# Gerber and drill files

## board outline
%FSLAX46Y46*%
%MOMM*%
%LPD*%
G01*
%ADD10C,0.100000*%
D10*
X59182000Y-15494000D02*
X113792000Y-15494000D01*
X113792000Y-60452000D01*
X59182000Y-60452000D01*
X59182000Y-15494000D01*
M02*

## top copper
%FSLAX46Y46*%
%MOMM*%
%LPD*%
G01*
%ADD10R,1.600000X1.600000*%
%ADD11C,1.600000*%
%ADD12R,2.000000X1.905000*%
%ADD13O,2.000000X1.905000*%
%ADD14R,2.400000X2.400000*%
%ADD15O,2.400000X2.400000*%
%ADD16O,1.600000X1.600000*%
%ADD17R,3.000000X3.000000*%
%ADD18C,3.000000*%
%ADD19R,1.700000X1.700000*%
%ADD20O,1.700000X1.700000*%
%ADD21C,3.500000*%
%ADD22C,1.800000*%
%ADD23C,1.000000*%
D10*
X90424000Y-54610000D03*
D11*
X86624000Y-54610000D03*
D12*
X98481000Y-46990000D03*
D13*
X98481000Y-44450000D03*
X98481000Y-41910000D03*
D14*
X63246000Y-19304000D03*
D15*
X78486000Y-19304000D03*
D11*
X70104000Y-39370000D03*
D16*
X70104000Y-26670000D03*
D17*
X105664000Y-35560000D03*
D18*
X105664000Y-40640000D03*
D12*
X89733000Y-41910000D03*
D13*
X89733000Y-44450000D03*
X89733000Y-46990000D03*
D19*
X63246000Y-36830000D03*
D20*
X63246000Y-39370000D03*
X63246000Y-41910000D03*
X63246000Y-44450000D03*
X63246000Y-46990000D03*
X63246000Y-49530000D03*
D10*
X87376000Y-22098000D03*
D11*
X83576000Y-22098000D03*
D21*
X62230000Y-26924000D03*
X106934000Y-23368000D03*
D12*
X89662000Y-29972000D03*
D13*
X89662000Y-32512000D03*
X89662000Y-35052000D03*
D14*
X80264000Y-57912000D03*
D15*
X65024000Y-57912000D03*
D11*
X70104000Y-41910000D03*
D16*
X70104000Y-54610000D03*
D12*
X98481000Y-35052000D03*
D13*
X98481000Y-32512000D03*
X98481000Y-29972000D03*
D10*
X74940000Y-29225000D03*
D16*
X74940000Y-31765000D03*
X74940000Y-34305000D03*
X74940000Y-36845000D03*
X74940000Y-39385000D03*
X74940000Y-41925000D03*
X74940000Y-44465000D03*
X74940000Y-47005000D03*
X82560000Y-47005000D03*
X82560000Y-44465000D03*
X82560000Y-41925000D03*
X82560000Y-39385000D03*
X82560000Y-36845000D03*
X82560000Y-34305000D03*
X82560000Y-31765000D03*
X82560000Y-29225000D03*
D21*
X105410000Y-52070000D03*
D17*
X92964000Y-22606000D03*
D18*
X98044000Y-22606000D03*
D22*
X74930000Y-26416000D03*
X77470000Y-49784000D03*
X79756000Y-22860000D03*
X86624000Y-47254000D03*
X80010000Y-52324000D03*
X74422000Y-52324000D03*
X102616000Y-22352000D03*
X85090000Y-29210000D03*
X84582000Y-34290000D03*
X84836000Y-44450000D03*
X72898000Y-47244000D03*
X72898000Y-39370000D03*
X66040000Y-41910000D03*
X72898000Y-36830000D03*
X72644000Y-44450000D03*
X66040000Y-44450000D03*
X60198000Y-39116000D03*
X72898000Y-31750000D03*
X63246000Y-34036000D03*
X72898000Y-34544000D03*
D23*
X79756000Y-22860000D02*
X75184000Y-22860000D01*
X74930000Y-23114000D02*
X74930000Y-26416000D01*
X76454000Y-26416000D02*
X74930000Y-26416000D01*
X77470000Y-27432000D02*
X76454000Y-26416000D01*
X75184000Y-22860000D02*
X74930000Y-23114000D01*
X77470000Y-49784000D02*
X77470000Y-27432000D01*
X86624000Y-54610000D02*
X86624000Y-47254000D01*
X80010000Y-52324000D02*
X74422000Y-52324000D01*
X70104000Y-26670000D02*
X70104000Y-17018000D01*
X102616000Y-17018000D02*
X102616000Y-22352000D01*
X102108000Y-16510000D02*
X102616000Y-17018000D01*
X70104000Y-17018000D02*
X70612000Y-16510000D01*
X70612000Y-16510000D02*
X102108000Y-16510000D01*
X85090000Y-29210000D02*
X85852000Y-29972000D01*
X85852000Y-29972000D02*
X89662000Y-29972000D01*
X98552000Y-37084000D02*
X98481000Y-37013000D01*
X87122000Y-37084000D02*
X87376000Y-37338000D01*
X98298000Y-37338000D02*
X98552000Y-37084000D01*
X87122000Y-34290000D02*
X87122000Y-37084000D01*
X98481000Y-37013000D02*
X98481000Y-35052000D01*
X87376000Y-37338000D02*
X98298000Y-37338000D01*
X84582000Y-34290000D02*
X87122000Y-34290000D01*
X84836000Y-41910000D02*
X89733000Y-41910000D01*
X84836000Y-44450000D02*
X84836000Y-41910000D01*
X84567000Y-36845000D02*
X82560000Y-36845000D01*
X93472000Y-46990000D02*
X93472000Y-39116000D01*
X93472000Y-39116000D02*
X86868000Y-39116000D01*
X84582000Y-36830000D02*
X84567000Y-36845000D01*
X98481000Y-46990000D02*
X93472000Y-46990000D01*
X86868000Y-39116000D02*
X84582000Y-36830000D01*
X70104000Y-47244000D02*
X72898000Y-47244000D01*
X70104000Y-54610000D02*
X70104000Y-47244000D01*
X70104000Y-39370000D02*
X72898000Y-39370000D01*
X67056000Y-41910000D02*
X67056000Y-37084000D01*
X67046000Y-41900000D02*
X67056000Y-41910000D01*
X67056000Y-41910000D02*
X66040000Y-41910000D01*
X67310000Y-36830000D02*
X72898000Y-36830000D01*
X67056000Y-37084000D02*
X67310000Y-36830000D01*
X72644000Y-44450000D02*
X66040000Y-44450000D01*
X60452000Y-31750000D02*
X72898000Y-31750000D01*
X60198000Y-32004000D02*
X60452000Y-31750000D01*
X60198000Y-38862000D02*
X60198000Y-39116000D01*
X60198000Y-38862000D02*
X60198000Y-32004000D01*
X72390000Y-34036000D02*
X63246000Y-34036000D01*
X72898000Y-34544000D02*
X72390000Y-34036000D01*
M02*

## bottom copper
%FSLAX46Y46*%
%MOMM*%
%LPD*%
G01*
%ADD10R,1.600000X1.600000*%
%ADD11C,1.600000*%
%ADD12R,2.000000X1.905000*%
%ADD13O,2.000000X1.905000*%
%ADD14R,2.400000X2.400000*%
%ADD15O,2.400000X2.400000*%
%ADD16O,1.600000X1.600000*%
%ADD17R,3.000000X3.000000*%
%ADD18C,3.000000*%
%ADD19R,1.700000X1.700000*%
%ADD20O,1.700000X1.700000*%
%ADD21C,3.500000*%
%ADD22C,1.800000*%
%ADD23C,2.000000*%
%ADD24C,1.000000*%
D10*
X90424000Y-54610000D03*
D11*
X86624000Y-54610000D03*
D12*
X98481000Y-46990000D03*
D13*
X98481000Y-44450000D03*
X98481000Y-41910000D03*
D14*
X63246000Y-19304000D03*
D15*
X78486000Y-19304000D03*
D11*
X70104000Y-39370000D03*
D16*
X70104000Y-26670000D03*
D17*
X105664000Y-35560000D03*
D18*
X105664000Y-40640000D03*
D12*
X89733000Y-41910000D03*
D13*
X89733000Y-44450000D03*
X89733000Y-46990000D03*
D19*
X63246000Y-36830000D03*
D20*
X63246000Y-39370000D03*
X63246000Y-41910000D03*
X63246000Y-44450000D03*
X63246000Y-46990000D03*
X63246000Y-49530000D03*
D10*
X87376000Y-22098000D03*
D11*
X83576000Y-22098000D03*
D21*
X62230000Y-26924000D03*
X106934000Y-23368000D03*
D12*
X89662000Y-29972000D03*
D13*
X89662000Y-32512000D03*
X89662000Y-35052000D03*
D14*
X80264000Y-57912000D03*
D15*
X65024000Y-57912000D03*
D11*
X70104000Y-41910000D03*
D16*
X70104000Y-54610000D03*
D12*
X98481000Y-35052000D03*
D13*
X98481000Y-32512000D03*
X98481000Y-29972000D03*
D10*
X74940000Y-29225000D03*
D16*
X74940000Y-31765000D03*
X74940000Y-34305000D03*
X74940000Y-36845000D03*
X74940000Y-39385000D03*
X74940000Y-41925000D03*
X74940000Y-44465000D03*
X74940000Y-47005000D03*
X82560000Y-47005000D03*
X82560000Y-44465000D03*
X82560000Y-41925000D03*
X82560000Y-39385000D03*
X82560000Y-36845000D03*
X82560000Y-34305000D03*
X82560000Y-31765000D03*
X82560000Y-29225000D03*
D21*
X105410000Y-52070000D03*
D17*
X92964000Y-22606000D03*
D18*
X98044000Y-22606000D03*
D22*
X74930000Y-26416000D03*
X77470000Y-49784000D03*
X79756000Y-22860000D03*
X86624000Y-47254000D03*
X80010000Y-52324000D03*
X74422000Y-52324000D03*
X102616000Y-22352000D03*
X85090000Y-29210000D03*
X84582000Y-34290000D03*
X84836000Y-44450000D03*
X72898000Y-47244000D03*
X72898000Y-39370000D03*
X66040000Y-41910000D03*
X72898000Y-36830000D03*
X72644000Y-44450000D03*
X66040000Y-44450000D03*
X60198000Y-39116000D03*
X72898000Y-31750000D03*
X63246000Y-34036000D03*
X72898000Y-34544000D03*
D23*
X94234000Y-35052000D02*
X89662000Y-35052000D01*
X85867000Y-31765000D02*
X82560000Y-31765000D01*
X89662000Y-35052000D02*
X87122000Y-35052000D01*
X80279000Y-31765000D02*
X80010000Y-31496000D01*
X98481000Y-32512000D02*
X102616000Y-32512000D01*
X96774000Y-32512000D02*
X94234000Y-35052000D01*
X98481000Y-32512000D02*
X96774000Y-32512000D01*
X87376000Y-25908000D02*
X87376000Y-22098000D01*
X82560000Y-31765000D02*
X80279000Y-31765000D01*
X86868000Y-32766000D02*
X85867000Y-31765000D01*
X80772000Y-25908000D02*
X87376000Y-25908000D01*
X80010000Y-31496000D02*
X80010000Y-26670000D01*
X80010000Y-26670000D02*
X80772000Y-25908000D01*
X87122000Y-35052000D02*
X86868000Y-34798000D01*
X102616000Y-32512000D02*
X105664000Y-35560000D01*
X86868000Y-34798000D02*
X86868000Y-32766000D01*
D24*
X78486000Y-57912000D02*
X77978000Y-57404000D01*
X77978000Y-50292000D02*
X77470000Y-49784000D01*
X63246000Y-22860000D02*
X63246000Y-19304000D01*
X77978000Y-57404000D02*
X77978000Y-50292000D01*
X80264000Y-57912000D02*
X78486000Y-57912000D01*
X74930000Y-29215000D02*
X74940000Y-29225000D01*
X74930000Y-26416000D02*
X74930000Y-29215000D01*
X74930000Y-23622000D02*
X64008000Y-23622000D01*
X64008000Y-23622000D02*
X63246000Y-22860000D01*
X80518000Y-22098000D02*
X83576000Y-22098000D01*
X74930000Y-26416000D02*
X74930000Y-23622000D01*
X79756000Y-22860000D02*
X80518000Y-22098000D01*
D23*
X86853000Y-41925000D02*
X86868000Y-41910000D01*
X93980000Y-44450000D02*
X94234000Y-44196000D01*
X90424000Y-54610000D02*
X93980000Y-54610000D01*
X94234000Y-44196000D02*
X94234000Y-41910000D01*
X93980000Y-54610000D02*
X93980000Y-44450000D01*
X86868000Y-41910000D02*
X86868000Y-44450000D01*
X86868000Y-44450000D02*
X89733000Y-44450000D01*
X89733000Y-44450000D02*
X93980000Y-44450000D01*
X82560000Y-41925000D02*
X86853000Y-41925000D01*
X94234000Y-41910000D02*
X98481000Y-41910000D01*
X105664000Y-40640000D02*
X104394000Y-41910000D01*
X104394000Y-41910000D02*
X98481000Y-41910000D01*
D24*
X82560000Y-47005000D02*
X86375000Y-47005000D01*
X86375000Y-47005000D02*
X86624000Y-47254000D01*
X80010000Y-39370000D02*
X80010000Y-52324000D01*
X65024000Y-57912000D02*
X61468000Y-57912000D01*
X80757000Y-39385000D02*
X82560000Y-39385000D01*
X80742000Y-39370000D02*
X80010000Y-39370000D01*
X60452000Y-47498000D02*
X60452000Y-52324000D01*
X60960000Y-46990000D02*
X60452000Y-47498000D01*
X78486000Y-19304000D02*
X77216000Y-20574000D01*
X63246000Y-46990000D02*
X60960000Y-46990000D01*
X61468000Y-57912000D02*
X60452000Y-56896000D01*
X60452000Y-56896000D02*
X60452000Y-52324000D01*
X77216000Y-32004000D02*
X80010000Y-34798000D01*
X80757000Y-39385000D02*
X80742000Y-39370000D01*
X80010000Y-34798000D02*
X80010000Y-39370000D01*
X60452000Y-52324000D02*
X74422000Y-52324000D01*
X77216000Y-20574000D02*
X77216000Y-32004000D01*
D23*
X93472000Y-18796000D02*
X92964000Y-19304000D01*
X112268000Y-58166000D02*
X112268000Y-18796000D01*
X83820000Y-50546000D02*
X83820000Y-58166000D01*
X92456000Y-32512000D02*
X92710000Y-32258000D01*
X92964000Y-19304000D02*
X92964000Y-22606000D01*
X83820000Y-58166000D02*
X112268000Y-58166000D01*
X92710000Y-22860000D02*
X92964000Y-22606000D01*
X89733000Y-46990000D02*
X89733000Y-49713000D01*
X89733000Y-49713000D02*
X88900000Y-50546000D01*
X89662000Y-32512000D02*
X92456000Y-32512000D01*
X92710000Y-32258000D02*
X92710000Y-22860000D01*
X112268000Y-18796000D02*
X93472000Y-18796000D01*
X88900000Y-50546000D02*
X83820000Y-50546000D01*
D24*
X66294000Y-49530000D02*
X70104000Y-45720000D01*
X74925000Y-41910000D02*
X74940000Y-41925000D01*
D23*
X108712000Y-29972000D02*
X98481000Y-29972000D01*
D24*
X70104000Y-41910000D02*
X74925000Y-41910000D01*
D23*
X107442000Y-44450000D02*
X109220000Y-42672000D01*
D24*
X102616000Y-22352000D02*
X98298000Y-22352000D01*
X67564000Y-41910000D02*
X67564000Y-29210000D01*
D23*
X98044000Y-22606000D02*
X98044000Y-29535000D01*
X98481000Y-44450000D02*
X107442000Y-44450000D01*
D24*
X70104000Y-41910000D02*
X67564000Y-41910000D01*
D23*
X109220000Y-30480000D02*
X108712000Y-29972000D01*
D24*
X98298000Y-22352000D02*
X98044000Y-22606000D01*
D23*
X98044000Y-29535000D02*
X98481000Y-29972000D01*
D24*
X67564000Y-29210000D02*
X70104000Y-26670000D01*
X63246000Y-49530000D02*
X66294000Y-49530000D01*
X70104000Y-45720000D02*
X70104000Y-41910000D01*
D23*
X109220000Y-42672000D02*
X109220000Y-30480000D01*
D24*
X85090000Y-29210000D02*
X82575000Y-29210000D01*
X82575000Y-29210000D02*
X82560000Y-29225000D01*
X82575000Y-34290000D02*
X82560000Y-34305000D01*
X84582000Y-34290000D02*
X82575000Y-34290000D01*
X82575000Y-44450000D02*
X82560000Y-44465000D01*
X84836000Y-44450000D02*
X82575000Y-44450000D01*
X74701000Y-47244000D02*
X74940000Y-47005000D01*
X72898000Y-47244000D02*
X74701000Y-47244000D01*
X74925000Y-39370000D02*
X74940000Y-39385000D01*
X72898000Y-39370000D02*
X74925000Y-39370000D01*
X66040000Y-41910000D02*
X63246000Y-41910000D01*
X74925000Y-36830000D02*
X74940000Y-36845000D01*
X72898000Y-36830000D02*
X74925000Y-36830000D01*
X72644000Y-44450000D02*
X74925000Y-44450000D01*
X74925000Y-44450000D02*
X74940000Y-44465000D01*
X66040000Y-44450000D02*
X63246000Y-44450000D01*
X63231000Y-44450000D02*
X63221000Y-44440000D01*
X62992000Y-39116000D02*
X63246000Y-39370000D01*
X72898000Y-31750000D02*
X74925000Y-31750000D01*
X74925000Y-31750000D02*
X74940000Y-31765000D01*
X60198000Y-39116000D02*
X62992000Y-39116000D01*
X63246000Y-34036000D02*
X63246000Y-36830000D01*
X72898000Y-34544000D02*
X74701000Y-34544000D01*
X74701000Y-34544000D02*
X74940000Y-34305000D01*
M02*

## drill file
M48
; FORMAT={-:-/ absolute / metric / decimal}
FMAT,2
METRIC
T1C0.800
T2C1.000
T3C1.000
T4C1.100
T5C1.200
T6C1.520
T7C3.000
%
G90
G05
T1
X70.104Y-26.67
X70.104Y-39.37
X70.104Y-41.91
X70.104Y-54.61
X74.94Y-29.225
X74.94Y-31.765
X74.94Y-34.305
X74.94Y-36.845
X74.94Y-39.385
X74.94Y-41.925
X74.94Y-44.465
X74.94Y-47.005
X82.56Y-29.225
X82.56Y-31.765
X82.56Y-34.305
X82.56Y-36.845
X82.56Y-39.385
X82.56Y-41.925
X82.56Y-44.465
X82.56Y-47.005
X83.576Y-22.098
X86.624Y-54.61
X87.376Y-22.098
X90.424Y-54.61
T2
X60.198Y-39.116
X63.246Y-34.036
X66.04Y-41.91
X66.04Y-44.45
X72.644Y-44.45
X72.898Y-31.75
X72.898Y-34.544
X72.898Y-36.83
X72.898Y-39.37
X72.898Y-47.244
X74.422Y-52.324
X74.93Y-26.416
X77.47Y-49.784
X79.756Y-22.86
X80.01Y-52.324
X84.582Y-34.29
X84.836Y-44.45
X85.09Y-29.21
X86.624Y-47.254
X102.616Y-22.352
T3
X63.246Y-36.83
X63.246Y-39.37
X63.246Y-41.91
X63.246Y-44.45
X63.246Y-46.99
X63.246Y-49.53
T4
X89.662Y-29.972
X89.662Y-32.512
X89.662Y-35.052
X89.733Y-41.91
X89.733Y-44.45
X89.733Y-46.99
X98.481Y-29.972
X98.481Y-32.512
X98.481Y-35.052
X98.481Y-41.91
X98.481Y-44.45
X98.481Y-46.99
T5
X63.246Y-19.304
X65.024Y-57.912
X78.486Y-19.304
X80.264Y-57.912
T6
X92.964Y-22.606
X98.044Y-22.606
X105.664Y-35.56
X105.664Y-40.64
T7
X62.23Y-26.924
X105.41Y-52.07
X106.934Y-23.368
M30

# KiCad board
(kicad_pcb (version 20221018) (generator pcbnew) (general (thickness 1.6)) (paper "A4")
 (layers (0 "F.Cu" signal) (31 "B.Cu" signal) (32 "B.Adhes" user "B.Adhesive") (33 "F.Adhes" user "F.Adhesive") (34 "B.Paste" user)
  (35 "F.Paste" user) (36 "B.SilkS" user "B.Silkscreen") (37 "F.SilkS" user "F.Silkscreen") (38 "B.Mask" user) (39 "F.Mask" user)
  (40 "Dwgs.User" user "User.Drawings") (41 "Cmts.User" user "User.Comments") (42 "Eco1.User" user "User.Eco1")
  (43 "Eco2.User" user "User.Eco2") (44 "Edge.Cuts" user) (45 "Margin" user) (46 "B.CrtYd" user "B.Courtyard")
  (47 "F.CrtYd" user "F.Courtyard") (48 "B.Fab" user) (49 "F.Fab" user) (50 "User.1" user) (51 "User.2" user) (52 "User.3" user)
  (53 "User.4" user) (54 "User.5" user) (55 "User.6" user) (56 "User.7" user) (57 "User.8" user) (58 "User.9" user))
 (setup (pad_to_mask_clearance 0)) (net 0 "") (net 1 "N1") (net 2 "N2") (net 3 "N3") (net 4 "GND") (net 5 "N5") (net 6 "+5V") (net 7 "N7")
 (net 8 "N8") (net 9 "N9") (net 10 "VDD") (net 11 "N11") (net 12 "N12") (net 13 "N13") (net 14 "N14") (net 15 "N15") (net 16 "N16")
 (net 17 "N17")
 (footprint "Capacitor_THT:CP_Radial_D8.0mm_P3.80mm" (layer "F.Cu") (at 90.424 54.61 180)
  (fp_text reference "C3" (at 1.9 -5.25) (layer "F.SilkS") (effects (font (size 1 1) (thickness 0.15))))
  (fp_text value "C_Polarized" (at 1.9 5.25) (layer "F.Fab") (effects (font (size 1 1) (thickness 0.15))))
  (pad "1" thru_hole rect (at 0 0 180) (size 1.6 1.6) (drill 0.8) (layers "*.Cu" "*.Mask") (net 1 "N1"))
  (pad "2" thru_hole circle (at 3.8 0 180) (size 1.6 1.6) (drill 0.8) (layers "*.Cu" "*.Mask") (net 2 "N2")))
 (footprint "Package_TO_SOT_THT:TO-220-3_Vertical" (layer "F.Cu") (at 98.481 46.99 90)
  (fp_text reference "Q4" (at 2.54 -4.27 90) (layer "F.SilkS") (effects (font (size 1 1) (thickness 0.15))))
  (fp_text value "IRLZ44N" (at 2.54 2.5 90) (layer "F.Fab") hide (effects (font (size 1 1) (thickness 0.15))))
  (pad "1" thru_hole rect (at 0 0 90) (size 1.905 2) (drill 1.1) (layers "*.Cu" "*.Mask") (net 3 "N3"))
  (pad "2" thru_hole oval (at 2.54 0 90) (size 1.905 2) (drill 1.1) (layers "*.Cu" "*.Mask") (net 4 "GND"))
  (pad "3" thru_hole oval (at 5.08 0 90) (size 1.905 2) (drill 1.1) (layers "*.Cu" "*.Mask") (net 1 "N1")))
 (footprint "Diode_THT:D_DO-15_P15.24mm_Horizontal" (layer "F.Cu") (at 63.246 19.304)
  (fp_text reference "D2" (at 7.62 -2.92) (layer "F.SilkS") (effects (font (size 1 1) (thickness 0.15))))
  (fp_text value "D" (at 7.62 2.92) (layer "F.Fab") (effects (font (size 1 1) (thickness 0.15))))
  (pad "1" thru_hole rect (at 0 0) (size 2.4 2.4) (drill 1.2) (layers "*.Cu" "*.Mask") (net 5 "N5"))
  (pad "2" thru_hole oval (at 15.24 0) (size 2.4 2.4) (drill 1.2) (layers "*.Cu" "*.Mask") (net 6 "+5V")))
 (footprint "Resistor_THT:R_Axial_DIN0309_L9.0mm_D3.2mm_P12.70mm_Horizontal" (layer "F.Cu") (at 70.104 39.37 90)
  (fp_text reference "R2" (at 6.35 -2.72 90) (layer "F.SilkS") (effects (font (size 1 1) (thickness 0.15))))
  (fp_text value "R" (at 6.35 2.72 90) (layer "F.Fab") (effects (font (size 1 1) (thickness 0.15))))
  (pad "1" thru_hole circle (at 0 0 90) (size 1.6 1.6) (drill 0.8) (layers "*.Cu" "*.Mask") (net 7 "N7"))
  (pad "2" thru_hole oval (at 12.7 0 90) (size 1.6 1.6) (drill 0.8) (layers "*.Cu" "*.Mask") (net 4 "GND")))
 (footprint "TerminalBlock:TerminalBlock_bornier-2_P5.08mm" (layer "F.Cu") (at 105.664 35.56 -90)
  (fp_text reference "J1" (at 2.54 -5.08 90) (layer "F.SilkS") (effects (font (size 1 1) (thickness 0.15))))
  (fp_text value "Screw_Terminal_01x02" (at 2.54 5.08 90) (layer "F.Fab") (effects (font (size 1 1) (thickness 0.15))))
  (pad "1" thru_hole rect (at 0 0 270) (size 3 3) (drill 1.52) (layers "*.Cu" "*.Mask") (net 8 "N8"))
  (pad "2" thru_hole circle (at 5.08 0 270) (size 3 3) (drill 1.52) (layers "*.Cu" "*.Mask") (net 1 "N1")))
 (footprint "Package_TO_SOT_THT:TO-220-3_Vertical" (layer "F.Cu") (at 89.733 41.91 -90)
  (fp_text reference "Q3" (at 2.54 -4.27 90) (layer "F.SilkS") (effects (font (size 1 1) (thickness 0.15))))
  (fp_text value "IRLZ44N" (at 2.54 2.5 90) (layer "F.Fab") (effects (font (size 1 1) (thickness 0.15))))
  (pad "1" thru_hole rect (at 0 0 270) (size 1.905 2) (drill 1.1) (layers "*.Cu" "*.Mask") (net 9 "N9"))
  (pad "2" thru_hole oval (at 2.54 0 270) (size 1.905 2) (drill 1.1) (layers "*.Cu" "*.Mask") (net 1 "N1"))
  (pad "3" thru_hole oval (at 5.08 0 270) (size 1.905 2) (drill 1.1) (layers "*.Cu" "*.Mask") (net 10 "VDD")))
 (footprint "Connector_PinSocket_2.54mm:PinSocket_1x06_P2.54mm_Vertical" (layer "F.Cu") (at 63.246 36.83)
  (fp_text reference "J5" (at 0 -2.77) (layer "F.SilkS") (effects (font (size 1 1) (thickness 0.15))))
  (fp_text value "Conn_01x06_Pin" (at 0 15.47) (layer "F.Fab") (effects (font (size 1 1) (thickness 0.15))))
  (pad "1" thru_hole rect (at 0 0) (size 1.7 1.7) (drill 1) (layers "*.Cu" "*.Mask") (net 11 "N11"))
  (pad "2" thru_hole oval (at 0 2.54) (size 1.7 1.7) (drill 1) (layers "*.Cu" "*.Mask") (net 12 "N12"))
  (pad "3" thru_hole oval (at 0 5.08) (size 1.7 1.7) (drill 1) (layers "*.Cu" "*.Mask") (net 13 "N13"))
  (pad "4" thru_hole oval (at 0 7.62) (size 1.7 1.7) (drill 1) (layers "*.Cu" "*.Mask") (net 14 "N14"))
  (pad "5" thru_hole oval (at 0 10.16) (size 1.7 1.7) (drill 1) (layers "*.Cu" "*.Mask") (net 6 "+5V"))
  (pad "6" thru_hole oval (at 0 12.7) (size 1.7 1.7) (drill 1) (layers "*.Cu" "*.Mask") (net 4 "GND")))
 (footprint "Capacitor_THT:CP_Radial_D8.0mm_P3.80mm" (layer "F.Cu") (at 87.376 22.098 180)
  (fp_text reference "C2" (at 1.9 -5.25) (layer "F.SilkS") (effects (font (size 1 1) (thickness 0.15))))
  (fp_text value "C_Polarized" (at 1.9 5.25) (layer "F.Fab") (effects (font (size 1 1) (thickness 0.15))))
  (pad "1" thru_hole rect (at 0 0 180) (size 1.6 1.6) (drill 0.8) (layers "*.Cu" "*.Mask") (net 8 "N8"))
  (pad "2" thru_hole circle (at 3.8 0 180) (size 1.6 1.6) (drill 0.8) (layers "*.Cu" "*.Mask") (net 5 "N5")))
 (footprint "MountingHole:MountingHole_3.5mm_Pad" (layer "F.Cu") (at 62.23 26.924)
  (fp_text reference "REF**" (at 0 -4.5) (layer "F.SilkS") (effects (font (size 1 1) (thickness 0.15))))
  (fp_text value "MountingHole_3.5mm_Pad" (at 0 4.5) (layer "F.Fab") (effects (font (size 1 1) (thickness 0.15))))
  (pad "1" thru_hole circle (at 0 0) (size 3.5 3.5) (drill 3) (layers "*.Cu" "*.Mask")))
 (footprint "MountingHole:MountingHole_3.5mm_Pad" (layer "F.Cu") (at 106.934 23.368)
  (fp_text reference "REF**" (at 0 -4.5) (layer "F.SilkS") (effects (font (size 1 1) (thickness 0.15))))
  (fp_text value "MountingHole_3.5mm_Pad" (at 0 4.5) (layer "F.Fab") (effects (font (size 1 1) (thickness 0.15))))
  (pad "1" thru_hole circle (at 0 0) (size 3.5 3.5) (drill 3) (layers "*.Cu" "*.Mask")))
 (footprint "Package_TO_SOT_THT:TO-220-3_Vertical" (layer "F.Cu") (at 89.662 29.972 -90)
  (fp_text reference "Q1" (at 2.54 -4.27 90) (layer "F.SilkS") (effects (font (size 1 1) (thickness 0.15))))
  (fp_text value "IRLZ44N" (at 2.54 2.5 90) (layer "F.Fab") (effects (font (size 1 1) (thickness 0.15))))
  (pad "1" thru_hole rect (at 0 0 270) (size 1.905 2) (drill 1.1) (layers "*.Cu" "*.Mask") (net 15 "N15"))
  (pad "2" thru_hole oval (at 2.54 0 270) (size 1.905 2) (drill 1.1) (layers "*.Cu" "*.Mask") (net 10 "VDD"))
  (pad "3" thru_hole oval (at 5.08 0 270) (size 1.905 2) (drill 1.1) (layers "*.Cu" "*.Mask") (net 8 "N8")))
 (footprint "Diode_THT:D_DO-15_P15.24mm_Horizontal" (layer "F.Cu") (at 80.264 57.912 180)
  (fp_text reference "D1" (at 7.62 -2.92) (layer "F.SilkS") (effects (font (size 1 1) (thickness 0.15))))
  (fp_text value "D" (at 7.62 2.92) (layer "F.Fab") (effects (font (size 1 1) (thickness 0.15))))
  (pad "1" thru_hole rect (at 0 0 180) (size 2.4 2.4) (drill 1.2) (layers "*.Cu" "*.Mask") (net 5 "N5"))
  (pad "2" thru_hole oval (at 15.24 0 180) (size 2.4 2.4) (drill 1.2) (layers "*.Cu" "*.Mask") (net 6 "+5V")))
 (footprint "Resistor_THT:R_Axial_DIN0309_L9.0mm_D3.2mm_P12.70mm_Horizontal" (layer "F.Cu") (at 70.104 41.91 -90)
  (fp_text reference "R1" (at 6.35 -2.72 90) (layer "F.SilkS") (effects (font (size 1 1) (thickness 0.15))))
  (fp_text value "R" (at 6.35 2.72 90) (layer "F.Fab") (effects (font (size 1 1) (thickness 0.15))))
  (pad "1" thru_hole circle (at 0 0 270) (size 1.6 1.6) (drill 0.8) (layers "*.Cu" "*.Mask") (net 4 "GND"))
  (pad "2" thru_hole oval (at 12.7 0 270) (size 1.6 1.6) (drill 0.8) (layers "*.Cu" "*.Mask") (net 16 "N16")))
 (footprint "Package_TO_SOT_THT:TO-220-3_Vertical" (layer "F.Cu") (at 98.481 35.052 90)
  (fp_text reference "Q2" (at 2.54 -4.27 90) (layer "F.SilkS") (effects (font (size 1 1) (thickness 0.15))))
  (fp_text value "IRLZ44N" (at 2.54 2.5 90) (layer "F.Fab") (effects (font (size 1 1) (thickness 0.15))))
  (pad "1" thru_hole rect (at 0 0 90) (size 1.905 2) (drill 1.1) (layers "*.Cu" "*.Mask") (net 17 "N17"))
  (pad "2" thru_hole oval (at 2.54 0 90) (size 1.905 2) (drill 1.1) (layers "*.Cu" "*.Mask") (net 8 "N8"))
  (pad "3" thru_hole oval (at 5.08 0 90) (size 1.905 2) (drill 1.1) (layers "*.Cu" "*.Mask") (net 4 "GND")))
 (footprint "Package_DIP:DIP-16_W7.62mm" (layer "F.Cu") (at 74.94 29.225)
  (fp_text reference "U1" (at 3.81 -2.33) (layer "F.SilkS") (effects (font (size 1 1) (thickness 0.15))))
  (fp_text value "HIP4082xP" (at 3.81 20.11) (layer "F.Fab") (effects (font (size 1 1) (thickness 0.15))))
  (pad "1" thru_hole rect (at 0 0) (size 1.6 1.6) (drill 0.8) (layers "*.Cu" "*.Mask") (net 5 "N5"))
  (pad "2" thru_hole oval (at 0 2.54) (size 1.6 1.6) (drill 0.8) (layers "*.Cu" "*.Mask") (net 12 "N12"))
  (pad "3" thru_hole oval (at 0 5.08) (size 1.6 1.6) (drill 0.8) (layers "*.Cu" "*.Mask") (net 11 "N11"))
  (pad "4" thru_hole oval (at 0 7.62) (size 1.6 1.6) (drill 0.8) (layers "*.Cu" "*.Mask") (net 13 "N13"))
  (pad "5" thru_hole oval (at 0 10.16) (size 1.6 1.6) (drill 0.8) (layers "*.Cu" "*.Mask") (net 7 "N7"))
  (pad "6" thru_hole oval (at 0 12.7) (size 1.6 1.6) (drill 0.8) (layers "*.Cu" "*.Mask") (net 4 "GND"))
  (pad "7" thru_hole oval (at 0 15.24) (size 1.6 1.6) (drill 0.8) (layers "*.Cu" "*.Mask") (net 14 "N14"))
  (pad "8" thru_hole oval (at 0 17.78) (size 1.6 1.6) (drill 0.8) (layers "*.Cu" "*.Mask") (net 16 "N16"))
  (pad "9" thru_hole oval (at 7.62 17.78) (size 1.6 1.6) (drill 0.8) (layers "*.Cu" "*.Mask") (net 2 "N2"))
  (pad "10" thru_hole oval (at 7.62 15.24) (size 1.6 1.6) (drill 0.8) (layers "*.Cu" "*.Mask") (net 9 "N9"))
  (pad "11" thru_hole oval (at 7.62 12.7) (size 1.6 1.6) (drill 0.8) (layers "*.Cu" "*.Mask") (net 1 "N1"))
  (pad "12" thru_hole oval (at 7.62 10.16) (size 1.6 1.6) (drill 0.8) (layers "*.Cu" "*.Mask") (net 6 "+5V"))
  (pad "13" thru_hole oval (at 7.62 7.62) (size 1.6 1.6) (drill 0.8) (layers "*.Cu" "*.Mask") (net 3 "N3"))
  (pad "14" thru_hole oval (at 7.62 5.08) (size 1.6 1.6) (drill 0.8) (layers "*.Cu" "*.Mask") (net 17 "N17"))
  (pad "15" thru_hole oval (at 7.62 2.54) (size 1.6 1.6) (drill 0.8) (layers "*.Cu" "*.Mask") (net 8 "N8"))
  (pad "16" thru_hole oval (at 7.62 0) (size 1.6 1.6) (drill 0.8) (layers "*.Cu" "*.Mask") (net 15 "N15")))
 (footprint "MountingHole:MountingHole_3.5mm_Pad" (layer "F.Cu") (at 105.41 52.07)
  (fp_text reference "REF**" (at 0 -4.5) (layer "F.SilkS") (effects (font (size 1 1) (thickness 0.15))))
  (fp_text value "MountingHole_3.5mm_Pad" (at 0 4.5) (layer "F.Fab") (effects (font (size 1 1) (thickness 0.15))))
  (pad "1" thru_hole circle (at 0 0) (size 3.5 3.5) (drill 3) (layers "*.Cu" "*.Mask")))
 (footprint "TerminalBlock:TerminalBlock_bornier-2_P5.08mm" (layer "F.Cu") (at 92.964 22.606)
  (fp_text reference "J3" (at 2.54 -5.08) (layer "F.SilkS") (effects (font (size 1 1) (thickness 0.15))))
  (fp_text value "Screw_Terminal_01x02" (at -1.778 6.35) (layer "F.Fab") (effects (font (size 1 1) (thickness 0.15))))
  (pad "1" thru_hole rect (at 0 0) (size 3 3) (drill 1.52) (layers "*.Cu" "*.Mask") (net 10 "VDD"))
  (pad "2" thru_hole circle (at 5.08 0) (size 3 3) (drill 1.52) (layers "*.Cu" "*.Mask") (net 4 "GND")))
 (gr_rect (start 59.182 15.494) (end 113.792 60.452) (stroke (width 0.1) (type default)) (fill none) (layer "Edge.Cuts"))
 (segment (start 94.234 35.052) (end 89.662 35.052) (width 2) (layer "B.Cu") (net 8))
 (segment (start 85.867 31.765) (end 82.56 31.765) (width 2) (layer "B.Cu") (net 8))
 (segment (start 89.662 35.052) (end 87.122 35.052) (width 2) (layer "B.Cu") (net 8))
 (segment (start 80.279 31.765) (end 80.01 31.496) (width 2) (layer "B.Cu") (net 8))
 (segment (start 98.481 32.512) (end 102.616 32.512) (width 2) (layer "B.Cu") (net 8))
 (segment (start 96.774 32.512) (end 94.234 35.052) (width 2) (layer "B.Cu") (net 8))
 (segment (start 98.481 32.512) (end 96.774 32.512) (width 2) (layer "B.Cu") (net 8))
 (segment (start 87.376 25.908) (end 87.376 22.098) (width 2) (layer "B.Cu") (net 8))
 (segment (start 82.56 31.765) (end 80.279 31.765) (width 2) (layer "B.Cu") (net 8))
 (segment (start 86.868 32.766) (end 85.867 31.765) (width 2) (layer "B.Cu") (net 8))
 (segment (start 80.772 25.908) (end 87.376 25.908) (width 2) (layer "B.Cu") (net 8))
 (segment (start 80.01 31.496) (end 80.01 26.67) (width 2) (layer "B.Cu") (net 8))
 (segment (start 80.01 26.67) (end 80.772 25.908) (width 2) (layer "B.Cu") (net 8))
 (segment (start 87.122 35.052) (end 86.868 34.798) (width 2) (layer "B.Cu") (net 8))
 (segment (start 102.616 32.512) (end 105.664 35.56) (width 2) (layer "B.Cu") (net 8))
 (segment (start 86.868 34.798) (end 86.868 32.766) (width 2) (layer "B.Cu") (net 8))
 (segment (start 79.756 22.86) (end 75.184 22.86) (width 1) (layer "F.Cu") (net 5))
 (segment (start 74.93 23.114) (end 74.93 26.416) (width 1) (layer "F.Cu") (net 5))
 (segment (start 76.454 26.416) (end 74.93 26.416) (width 1) (layer "F.Cu") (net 5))
 (segment (start 77.47 27.432) (end 76.454 26.416) (width 1) (layer "F.Cu") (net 5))
 (segment (start 75.184 22.86) (end 74.93 23.114) (width 1) (layer "F.Cu") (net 5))
 (segment (start 77.47 49.784) (end 77.47 27.432) (width 1) (layer "F.Cu") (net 5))
 (via (at 74.93 26.416) (size 1.8) (drill 1) (layers "F.Cu" "B.Cu") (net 5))
 (via (at 77.47 49.784) (size 1.8) (drill 1) (layers "F.Cu" "B.Cu") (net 5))
 (via (at 79.756 22.86) (size 1.8) (drill 1) (layers "F.Cu" "B.Cu") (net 5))
 (segment (start 78.486 57.912) (end 77.978 57.404) (width 1) (layer "B.Cu") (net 5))
 (segment (start 77.978 50.292) (end 77.47 49.784) (width 1) (layer "B.Cu") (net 5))
 (segment (start 63.246 22.86) (end 63.246 19.304) (width 1) (layer "B.Cu") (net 5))
 (segment (start 77.978 57.404) (end 77.978 50.292) (width 1) (layer "B.Cu") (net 5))
 (segment (start 80.264 57.912) (end 78.486 57.912) (width 1) (layer "B.Cu") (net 5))
 (segment (start 74.93 29.215) (end 74.94 29.225) (width 1) (layer "B.Cu") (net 5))
 (segment (start 74.93 26.416) (end 74.93 29.215) (width 1) (layer "B.Cu") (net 5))
 (segment (start 74.93 23.622) (end 64.008 23.622) (width 1) (layer "B.Cu") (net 5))
 (segment (start 64.008 23.622) (end 63.246 22.86) (width 1) (layer "B.Cu") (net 5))
 (segment (start 80.518 22.098) (end 83.576 22.098) (width 1) (layer "B.Cu") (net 5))
 (segment (start 74.93 26.416) (end 74.93 23.622) (width 1) (layer "B.Cu") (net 5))
 (segment (start 79.756 22.86) (end 80.518 22.098) (width 1) (layer "B.Cu") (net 5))
 (segment (start 86.853 41.925) (end 86.868 41.91) (width 2) (layer "B.Cu") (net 1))
 (segment (start 93.98 44.45) (end 94.234 44.196) (width 2) (layer "B.Cu") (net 1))
 (segment (start 90.424 54.61) (end 93.98 54.61) (width 2) (layer "B.Cu") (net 1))
 (segment (start 94.234 44.196) (end 94.234 41.91) (width 2) (layer "B.Cu") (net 1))
 (segment (start 93.98 54.61) (end 93.98 44.45) (width 2) (layer "B.Cu") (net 1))
 (segment (start 86.868 41.91) (end 86.868 44.45) (width 2) (layer "B.Cu") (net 1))
 (segment (start 86.868 44.45) (end 89.733 44.45) (width 2) (layer "B.Cu") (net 1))
 (segment (start 89.733 44.45) (end 93.98 44.45) (width 2) (layer "B.Cu") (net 1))
 (segment (start 82.56 41.925) (end 86.853 41.925) (width 2) (layer "B.Cu") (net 1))
 (segment (start 94.234 41.91) (end 98.481 41.91) (width 2) (layer "B.Cu") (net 1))
 (segment (start 105.664 40.64) (end 104.394 41.91) (width 2) (layer "B.Cu") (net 1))
 (segment (start 104.394 41.91) (end 98.481 41.91) (width 2) (layer "B.Cu") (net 1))
 (segment (start 86.624 54.61) (end 86.624 47.254) (width 1) (layer "F.Cu") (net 2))
 (via (at 86.624 47.254) (size 1.8) (drill 1) (layers "F.Cu" "B.Cu") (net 2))
 (segment (start 82.56 47.005) (end 86.375 47.005) (width 1) (layer "B.Cu") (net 2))
 (segment (start 86.375 47.005) (end 86.624 47.254) (width 1) (layer "B.Cu") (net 2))
 (segment (start 80.01 52.324) (end 74.422 52.324) (width 1) (layer "F.Cu") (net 6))
 (via (at 80.01 52.324) (size 1.8) (drill 1) (layers "F.Cu" "B.Cu") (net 6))
 (via (at 74.422 52.324) (size 1.8) (drill 1) (layers "F.Cu" "B.Cu") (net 6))
 (segment (start 80.01 39.37) (end 80.01 52.324) (width 1) (layer "B.Cu") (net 6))
 (segment (start 65.024 57.912) (end 61.468 57.912) (width 1) (layer "B.Cu") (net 6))
 (segment (start 80.757 39.385) (end 82.56 39.385) (width 1) (layer "B.Cu") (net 6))
 (segment (start 80.742 39.37) (end 80.01 39.37) (width 1) (layer "B.Cu") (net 6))
 (segment (start 60.452 47.498) (end 60.452 52.324) (width 1) (layer "B.Cu") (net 6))
 (segment (start 60.96 46.99) (end 60.452 47.498) (width 1) (layer "B.Cu") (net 6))
 (segment (start 78.486 19.304) (end 77.216 20.574) (width 1) (layer "B.Cu") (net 6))
 (segment (start 63.246 46.99) (end 60.96 46.99) (width 1) (layer "B.Cu") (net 6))
 (segment (start 61.468 57.912) (end 60.452 56.896) (width 1) (layer "B.Cu") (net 6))
 (segment (start 60.452 56.896) (end 60.452 52.324) (width 1) (layer "B.Cu") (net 6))
 (segment (start 77.216 32.004) (end 80.01 34.798) (width 1) (layer "B.Cu") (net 6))
 (segment (start 80.757 39.385) (end 80.742 39.37) (width 1) (layer "B.Cu") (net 6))
 (segment (start 80.01 34.798) (end 80.01 39.37) (width 1) (layer "B.Cu") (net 6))
 (segment (start 60.452 52.324) (end 74.422 52.324) (width 1) (layer "B.Cu") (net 6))
 (segment (start 77.216 20.574) (end 77.216 32.004) (width 1) (layer "B.Cu") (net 6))
 (segment (start 93.472 18.796) (end 92.964 19.304) (width 2) (layer "B.Cu") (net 10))
 (segment (start 112.268 58.166) (end 112.268 18.796) (width 2) (layer "B.Cu") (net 10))
 (segment (start 83.82 50.546) (end 83.82 58.166) (width 2) (layer "B.Cu") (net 10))
 (segment (start 92.456 32.512) (end 92.71 32.258) (width 2) (layer "B.Cu") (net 10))
 (segment (start 92.964 19.304) (end 92.964 22.606) (width 2) (layer "B.Cu") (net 10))
 (segment (start 83.82 58.166) (end 112.268 58.166) (width 2) (layer "B.Cu") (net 10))
 (segment (start 92.71 22.86) (end 92.964 22.606) (width 2) (layer "B.Cu") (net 10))
 (segment (start 89.733 46.99) (end 89.733 49.713) (width 2) (layer "B.Cu") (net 10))
 (segment (start 89.733 49.713) (end 88.9 50.546) (width 2) (layer "B.Cu") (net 10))
 (segment (start 89.662 32.512) (end 92.456 32.512) (width 2) (layer "B.Cu") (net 10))
 (segment (start 92.71 32.258) (end 92.71 22.86) (width 2) (layer "B.Cu") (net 10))
 (segment (start 112.268 18.796) (end 93.472 18.796) (width 2) (layer "B.Cu") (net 10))
 (segment (start 88.9 50.546) (end 83.82 50.546) (width 2) (layer "B.Cu") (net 10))
 (segment (start 70.104 26.67) (end 70.104 17.018) (width 1) (layer "F.Cu") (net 4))
 (segment (start 102.616 17.018) (end 102.616 22.352) (width 1) (layer "F.Cu") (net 4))
 (segment (start 102.108 16.51) (end 102.616 17.018) (width 1) (layer "F.Cu") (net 4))
 (segment (start 70.104 17.018) (end 70.612 16.51) (width 1) (layer "F.Cu") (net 4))
 (segment (start 70.612 16.51) (end 102.108 16.51) (width 1) (layer "F.Cu") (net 4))
 (via (at 102.616 22.352) (size 1.8) (drill 1) (layers "F.Cu" "B.Cu") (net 4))
 (segment (start 66.294 49.53) (end 70.104 45.72) (width 1) (layer "B.Cu") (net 4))
 (segment (start 74.925 41.91) (end 74.94 41.925) (width 1) (layer "B.Cu") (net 4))
 (segment (start 108.712 29.972) (end 98.481 29.972) (width 2) (layer "B.Cu") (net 4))
 (segment (start 70.104 41.91) (end 74.925 41.91) (width 1) (layer "B.Cu") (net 4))
 (segment (start 107.442 44.45) (end 109.22 42.672) (width 2) (layer "B.Cu") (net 4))
 (segment (start 102.616 22.352) (end 98.298 22.352) (width 1) (layer "B.Cu") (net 4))
 (segment (start 67.564 41.91) (end 67.564 29.21) (width 1) (layer "B.Cu") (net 4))
 (segment (start 98.044 22.606) (end 98.044 29.535) (width 2) (layer "B.Cu") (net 4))
 (segment (start 98.481 44.45) (end 107.442 44.45) (width 2) (layer "B.Cu") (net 4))
 (segment (start 70.104 41.91) (end 67.564 41.91) (width 1) (layer "B.Cu") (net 4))
 (segment (start 109.22 30.48) (end 108.712 29.972) (width 2) (layer "B.Cu") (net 4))
 (segment (start 98.298 22.352) (end 98.044 22.606) (width 1) (layer "B.Cu") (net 4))
 (segment (start 98.044 29.535) (end 98.481 29.972) (width 2) (layer "B.Cu") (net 4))
 (segment (start 67.564 29.21) (end 70.104 26.67) (width 1) (layer "B.Cu") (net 4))
 (segment (start 63.246 49.53) (end 66.294 49.53) (width 1) (layer "B.Cu") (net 4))
 (segment (start 70.104 45.72) (end 70.104 41.91) (width 1) (layer "B.Cu") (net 4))
 (segment (start 109.22 42.672) (end 109.22 30.48) (width 2) (layer "B.Cu") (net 4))
 (segment (start 85.09 29.21) (end 85.852 29.972) (width 1) (layer "F.Cu") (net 15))
 (segment (start 85.852 29.972) (end 89.662 29.972) (width 1) (layer "F.Cu") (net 15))
 (via (at 85.09 29.21) (size 1.8) (drill 1) (layers "F.Cu" "B.Cu") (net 15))
 (segment (start 85.09 29.21) (end 82.575 29.21) (width 1) (layer "B.Cu") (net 15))
 (segment (start 82.575 29.21) (end 82.56 29.225) (width 1) (layer "B.Cu") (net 15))
 (segment (start 98.552 37.084) (end 98.481 37.013) (width 1) (layer "F.Cu") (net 17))
 (segment (start 87.122 37.084) (end 87.376 37.338) (width 1) (layer "F.Cu") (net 17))
 (segment (start 98.298 37.338) (end 98.552 37.084) (width 1) (layer "F.Cu") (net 17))
 (segment (start 87.122 34.29) (end 87.122 37.084) (width 1) (layer "F.Cu") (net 17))
 (segment (start 98.481 37.013) (end 98.481 35.052) (width 1) (layer "F.Cu") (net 17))
 (segment (start 87.376 37.338) (end 98.298 37.338) (width 1) (layer "F.Cu") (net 17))
 (segment (start 84.582 34.29) (end 87.122 34.29) (width 1) (layer "F.Cu") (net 17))
 (via (at 84.582 34.29) (size 1.8) (drill 1) (layers "F.Cu" "B.Cu") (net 17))
 (segment (start 82.575 34.29) (end 82.56 34.305) (width 1) (layer "B.Cu") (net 17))
 (segment (start 84.582 34.29) (end 82.575 34.29) (width 1) (layer "B.Cu") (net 17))
 (segment (start 84.836 41.91) (end 89.733 41.91) (width 1) (layer "F.Cu") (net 9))
 (segment (start 84.836 44.45) (end 84.836 41.91) (width 1) (layer "F.Cu") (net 9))
 (via (at 84.836 44.45) (size 1.8) (drill 1) (layers "F.Cu" "B.Cu") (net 9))
 (segment (start 82.575 44.45) (end 82.56 44.465) (width 1) (layer "B.Cu") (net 9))
 (segment (start 84.836 44.45) (end 82.575 44.45) (width 1) (layer "B.Cu") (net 9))
 (segment (start 84.567 36.845) (end 82.56 36.845) (width 1) (layer "F.Cu") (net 3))
 (segment (start 93.472 46.99) (end 93.472 39.116) (width 1) (layer "F.Cu") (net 3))
 (segment (start 93.472 39.116) (end 86.868 39.116) (width 1) (layer "F.Cu") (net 3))
 (segment (start 84.582 36.83) (end 84.567 36.845) (width 1) (layer "F.Cu") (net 3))
 (segment (start 98.481 46.99) (end 93.472 46.99) (width 1) (layer "F.Cu") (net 3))
 (segment (start 86.868 39.116) (end 84.582 36.83) (width 1) (layer "F.Cu") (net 3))
 (segment (start 70.104 47.244) (end 72.898 47.244) (width 1) (layer "F.Cu") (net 16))
 (segment (start 70.104 54.61) (end 70.104 47.244) (width 1) (layer "F.Cu") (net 16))
 (via (at 72.898 47.244) (size 1.8) (drill 1) (layers "F.Cu" "B.Cu") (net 16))
 (segment (start 74.701 47.244) (end 74.94 47.005) (width 1) (layer "B.Cu") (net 16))
 (segment (start 72.898 47.244) (end 74.701 47.244) (width 1) (layer "B.Cu") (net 16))
 (segment (start 70.104 39.37) (end 72.898 39.37) (width 1) (layer "F.Cu") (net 7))
 (via (at 72.898 39.37) (size 1.8) (drill 1) (layers "F.Cu" "B.Cu") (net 7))
 (segment (start 74.925 39.37) (end 74.94 39.385) (width 1) (layer "B.Cu") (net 7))
 (segment (start 72.898 39.37) (end 74.925 39.37) (width 1) (layer "B.Cu") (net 7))
 (segment (start 67.056 41.91) (end 67.056 37.084) (width 1) (layer "F.Cu") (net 13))
 (segment (start 67.046 41.9) (end 67.056 41.91) (width 1) (layer "F.Cu") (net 13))
 (segment (start 67.056 41.91) (end 66.04 41.91) (width 1) (layer "F.Cu") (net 13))
 (segment (start 67.31 36.83) (end 72.898 36.83) (width 1) (layer "F.Cu") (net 13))
 (segment (start 67.056 37.084) (end 67.31 36.83) (width 1) (layer "F.Cu") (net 13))
 (via (at 66.04 41.91) (size 1.8) (drill 1) (layers "F.Cu" "B.Cu") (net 13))
 (via (at 72.898 36.83) (size 1.8) (drill 1) (layers "F.Cu" "B.Cu") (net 13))
 (segment (start 66.04 41.91) (end 63.246 41.91) (width 1) (layer "B.Cu") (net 13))
 (segment (start 74.925 36.83) (end 74.94 36.845) (width 1) (layer "B.Cu") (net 13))
 (segment (start 72.898 36.83) (end 74.925 36.83) (width 1) (layer "B.Cu") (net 13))
 (segment (start 72.644 44.45) (end 66.04 44.45) (width 1) (layer "F.Cu") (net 14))
 (via (at 72.644 44.45) (size 1.8) (drill 1) (layers "F.Cu" "B.Cu") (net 14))
 (via (at 66.04 44.45) (size 1.8) (drill 1) (layers "F.Cu" "B.Cu") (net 14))
 (segment (start 72.644 44.45) (end 74.925 44.45) (width 1) (layer "B.Cu") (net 14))
 (segment (start 74.925 44.45) (end 74.94 44.465) (width 1) (layer "B.Cu") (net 14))
 (segment (start 66.04 44.45) (end 63.246 44.45) (width 1) (layer "B.Cu") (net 14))
 (segment (start 63.231 44.45) (end 63.221 44.44) (width 1) (layer "B.Cu") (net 14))
 (segment (start 60.452 31.75) (end 72.898 31.75) (width 1) (layer "F.Cu") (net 12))
 (segment (start 60.198 32.004) (end 60.452 31.75) (width 1) (layer "F.Cu") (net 12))
 (segment (start 60.198 38.862) (end 60.198 39.116) (width 1) (layer "F.Cu") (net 12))
 (segment (start 60.198 38.862) (end 60.198 32.004) (width 1) (layer "F.Cu") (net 12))
 (via (at 60.198 39.116) (size 1.8) (drill 1) (layers "F.Cu" "B.Cu") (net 12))
 (via (at 72.898 31.75) (size 1.8) (drill 1) (layers "F.Cu" "B.Cu") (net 12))
 (segment (start 62.992 39.116) (end 63.246 39.37) (width 1) (layer "B.Cu") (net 12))
 (segment (start 72.898 31.75) (end 74.925 31.75) (width 1) (layer "B.Cu") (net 12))
 (segment (start 74.925 31.75) (end 74.94 31.765) (width 1) (layer "B.Cu") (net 12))
 (segment (start 60.198 39.116) (end 62.992 39.116) (width 1) (layer "B.Cu") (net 12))
 (segment (start 72.39 34.036) (end 63.246 34.036) (width 1) (layer "F.Cu") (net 11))
 (segment (start 72.898 34.544) (end 72.39 34.036) (width 1) (layer "F.Cu") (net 11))
 (via (at 63.246 34.036) (size 1.8) (drill 1) (layers "F.Cu" "B.Cu") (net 11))
 (via (at 72.898 34.544) (size 1.8) (drill 1) (layers "F.Cu" "B.Cu") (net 11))
 (segment (start 63.246 34.036) (end 63.246 36.83) (width 1) (layer "B.Cu") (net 11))
 (segment (start 72.898 34.544) (end 74.701 34.544) (width 1) (layer "B.Cu") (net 11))
 (segment (start 74.701 34.544) (end 74.94 34.305) (width 1) (layer "B.Cu") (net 11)))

